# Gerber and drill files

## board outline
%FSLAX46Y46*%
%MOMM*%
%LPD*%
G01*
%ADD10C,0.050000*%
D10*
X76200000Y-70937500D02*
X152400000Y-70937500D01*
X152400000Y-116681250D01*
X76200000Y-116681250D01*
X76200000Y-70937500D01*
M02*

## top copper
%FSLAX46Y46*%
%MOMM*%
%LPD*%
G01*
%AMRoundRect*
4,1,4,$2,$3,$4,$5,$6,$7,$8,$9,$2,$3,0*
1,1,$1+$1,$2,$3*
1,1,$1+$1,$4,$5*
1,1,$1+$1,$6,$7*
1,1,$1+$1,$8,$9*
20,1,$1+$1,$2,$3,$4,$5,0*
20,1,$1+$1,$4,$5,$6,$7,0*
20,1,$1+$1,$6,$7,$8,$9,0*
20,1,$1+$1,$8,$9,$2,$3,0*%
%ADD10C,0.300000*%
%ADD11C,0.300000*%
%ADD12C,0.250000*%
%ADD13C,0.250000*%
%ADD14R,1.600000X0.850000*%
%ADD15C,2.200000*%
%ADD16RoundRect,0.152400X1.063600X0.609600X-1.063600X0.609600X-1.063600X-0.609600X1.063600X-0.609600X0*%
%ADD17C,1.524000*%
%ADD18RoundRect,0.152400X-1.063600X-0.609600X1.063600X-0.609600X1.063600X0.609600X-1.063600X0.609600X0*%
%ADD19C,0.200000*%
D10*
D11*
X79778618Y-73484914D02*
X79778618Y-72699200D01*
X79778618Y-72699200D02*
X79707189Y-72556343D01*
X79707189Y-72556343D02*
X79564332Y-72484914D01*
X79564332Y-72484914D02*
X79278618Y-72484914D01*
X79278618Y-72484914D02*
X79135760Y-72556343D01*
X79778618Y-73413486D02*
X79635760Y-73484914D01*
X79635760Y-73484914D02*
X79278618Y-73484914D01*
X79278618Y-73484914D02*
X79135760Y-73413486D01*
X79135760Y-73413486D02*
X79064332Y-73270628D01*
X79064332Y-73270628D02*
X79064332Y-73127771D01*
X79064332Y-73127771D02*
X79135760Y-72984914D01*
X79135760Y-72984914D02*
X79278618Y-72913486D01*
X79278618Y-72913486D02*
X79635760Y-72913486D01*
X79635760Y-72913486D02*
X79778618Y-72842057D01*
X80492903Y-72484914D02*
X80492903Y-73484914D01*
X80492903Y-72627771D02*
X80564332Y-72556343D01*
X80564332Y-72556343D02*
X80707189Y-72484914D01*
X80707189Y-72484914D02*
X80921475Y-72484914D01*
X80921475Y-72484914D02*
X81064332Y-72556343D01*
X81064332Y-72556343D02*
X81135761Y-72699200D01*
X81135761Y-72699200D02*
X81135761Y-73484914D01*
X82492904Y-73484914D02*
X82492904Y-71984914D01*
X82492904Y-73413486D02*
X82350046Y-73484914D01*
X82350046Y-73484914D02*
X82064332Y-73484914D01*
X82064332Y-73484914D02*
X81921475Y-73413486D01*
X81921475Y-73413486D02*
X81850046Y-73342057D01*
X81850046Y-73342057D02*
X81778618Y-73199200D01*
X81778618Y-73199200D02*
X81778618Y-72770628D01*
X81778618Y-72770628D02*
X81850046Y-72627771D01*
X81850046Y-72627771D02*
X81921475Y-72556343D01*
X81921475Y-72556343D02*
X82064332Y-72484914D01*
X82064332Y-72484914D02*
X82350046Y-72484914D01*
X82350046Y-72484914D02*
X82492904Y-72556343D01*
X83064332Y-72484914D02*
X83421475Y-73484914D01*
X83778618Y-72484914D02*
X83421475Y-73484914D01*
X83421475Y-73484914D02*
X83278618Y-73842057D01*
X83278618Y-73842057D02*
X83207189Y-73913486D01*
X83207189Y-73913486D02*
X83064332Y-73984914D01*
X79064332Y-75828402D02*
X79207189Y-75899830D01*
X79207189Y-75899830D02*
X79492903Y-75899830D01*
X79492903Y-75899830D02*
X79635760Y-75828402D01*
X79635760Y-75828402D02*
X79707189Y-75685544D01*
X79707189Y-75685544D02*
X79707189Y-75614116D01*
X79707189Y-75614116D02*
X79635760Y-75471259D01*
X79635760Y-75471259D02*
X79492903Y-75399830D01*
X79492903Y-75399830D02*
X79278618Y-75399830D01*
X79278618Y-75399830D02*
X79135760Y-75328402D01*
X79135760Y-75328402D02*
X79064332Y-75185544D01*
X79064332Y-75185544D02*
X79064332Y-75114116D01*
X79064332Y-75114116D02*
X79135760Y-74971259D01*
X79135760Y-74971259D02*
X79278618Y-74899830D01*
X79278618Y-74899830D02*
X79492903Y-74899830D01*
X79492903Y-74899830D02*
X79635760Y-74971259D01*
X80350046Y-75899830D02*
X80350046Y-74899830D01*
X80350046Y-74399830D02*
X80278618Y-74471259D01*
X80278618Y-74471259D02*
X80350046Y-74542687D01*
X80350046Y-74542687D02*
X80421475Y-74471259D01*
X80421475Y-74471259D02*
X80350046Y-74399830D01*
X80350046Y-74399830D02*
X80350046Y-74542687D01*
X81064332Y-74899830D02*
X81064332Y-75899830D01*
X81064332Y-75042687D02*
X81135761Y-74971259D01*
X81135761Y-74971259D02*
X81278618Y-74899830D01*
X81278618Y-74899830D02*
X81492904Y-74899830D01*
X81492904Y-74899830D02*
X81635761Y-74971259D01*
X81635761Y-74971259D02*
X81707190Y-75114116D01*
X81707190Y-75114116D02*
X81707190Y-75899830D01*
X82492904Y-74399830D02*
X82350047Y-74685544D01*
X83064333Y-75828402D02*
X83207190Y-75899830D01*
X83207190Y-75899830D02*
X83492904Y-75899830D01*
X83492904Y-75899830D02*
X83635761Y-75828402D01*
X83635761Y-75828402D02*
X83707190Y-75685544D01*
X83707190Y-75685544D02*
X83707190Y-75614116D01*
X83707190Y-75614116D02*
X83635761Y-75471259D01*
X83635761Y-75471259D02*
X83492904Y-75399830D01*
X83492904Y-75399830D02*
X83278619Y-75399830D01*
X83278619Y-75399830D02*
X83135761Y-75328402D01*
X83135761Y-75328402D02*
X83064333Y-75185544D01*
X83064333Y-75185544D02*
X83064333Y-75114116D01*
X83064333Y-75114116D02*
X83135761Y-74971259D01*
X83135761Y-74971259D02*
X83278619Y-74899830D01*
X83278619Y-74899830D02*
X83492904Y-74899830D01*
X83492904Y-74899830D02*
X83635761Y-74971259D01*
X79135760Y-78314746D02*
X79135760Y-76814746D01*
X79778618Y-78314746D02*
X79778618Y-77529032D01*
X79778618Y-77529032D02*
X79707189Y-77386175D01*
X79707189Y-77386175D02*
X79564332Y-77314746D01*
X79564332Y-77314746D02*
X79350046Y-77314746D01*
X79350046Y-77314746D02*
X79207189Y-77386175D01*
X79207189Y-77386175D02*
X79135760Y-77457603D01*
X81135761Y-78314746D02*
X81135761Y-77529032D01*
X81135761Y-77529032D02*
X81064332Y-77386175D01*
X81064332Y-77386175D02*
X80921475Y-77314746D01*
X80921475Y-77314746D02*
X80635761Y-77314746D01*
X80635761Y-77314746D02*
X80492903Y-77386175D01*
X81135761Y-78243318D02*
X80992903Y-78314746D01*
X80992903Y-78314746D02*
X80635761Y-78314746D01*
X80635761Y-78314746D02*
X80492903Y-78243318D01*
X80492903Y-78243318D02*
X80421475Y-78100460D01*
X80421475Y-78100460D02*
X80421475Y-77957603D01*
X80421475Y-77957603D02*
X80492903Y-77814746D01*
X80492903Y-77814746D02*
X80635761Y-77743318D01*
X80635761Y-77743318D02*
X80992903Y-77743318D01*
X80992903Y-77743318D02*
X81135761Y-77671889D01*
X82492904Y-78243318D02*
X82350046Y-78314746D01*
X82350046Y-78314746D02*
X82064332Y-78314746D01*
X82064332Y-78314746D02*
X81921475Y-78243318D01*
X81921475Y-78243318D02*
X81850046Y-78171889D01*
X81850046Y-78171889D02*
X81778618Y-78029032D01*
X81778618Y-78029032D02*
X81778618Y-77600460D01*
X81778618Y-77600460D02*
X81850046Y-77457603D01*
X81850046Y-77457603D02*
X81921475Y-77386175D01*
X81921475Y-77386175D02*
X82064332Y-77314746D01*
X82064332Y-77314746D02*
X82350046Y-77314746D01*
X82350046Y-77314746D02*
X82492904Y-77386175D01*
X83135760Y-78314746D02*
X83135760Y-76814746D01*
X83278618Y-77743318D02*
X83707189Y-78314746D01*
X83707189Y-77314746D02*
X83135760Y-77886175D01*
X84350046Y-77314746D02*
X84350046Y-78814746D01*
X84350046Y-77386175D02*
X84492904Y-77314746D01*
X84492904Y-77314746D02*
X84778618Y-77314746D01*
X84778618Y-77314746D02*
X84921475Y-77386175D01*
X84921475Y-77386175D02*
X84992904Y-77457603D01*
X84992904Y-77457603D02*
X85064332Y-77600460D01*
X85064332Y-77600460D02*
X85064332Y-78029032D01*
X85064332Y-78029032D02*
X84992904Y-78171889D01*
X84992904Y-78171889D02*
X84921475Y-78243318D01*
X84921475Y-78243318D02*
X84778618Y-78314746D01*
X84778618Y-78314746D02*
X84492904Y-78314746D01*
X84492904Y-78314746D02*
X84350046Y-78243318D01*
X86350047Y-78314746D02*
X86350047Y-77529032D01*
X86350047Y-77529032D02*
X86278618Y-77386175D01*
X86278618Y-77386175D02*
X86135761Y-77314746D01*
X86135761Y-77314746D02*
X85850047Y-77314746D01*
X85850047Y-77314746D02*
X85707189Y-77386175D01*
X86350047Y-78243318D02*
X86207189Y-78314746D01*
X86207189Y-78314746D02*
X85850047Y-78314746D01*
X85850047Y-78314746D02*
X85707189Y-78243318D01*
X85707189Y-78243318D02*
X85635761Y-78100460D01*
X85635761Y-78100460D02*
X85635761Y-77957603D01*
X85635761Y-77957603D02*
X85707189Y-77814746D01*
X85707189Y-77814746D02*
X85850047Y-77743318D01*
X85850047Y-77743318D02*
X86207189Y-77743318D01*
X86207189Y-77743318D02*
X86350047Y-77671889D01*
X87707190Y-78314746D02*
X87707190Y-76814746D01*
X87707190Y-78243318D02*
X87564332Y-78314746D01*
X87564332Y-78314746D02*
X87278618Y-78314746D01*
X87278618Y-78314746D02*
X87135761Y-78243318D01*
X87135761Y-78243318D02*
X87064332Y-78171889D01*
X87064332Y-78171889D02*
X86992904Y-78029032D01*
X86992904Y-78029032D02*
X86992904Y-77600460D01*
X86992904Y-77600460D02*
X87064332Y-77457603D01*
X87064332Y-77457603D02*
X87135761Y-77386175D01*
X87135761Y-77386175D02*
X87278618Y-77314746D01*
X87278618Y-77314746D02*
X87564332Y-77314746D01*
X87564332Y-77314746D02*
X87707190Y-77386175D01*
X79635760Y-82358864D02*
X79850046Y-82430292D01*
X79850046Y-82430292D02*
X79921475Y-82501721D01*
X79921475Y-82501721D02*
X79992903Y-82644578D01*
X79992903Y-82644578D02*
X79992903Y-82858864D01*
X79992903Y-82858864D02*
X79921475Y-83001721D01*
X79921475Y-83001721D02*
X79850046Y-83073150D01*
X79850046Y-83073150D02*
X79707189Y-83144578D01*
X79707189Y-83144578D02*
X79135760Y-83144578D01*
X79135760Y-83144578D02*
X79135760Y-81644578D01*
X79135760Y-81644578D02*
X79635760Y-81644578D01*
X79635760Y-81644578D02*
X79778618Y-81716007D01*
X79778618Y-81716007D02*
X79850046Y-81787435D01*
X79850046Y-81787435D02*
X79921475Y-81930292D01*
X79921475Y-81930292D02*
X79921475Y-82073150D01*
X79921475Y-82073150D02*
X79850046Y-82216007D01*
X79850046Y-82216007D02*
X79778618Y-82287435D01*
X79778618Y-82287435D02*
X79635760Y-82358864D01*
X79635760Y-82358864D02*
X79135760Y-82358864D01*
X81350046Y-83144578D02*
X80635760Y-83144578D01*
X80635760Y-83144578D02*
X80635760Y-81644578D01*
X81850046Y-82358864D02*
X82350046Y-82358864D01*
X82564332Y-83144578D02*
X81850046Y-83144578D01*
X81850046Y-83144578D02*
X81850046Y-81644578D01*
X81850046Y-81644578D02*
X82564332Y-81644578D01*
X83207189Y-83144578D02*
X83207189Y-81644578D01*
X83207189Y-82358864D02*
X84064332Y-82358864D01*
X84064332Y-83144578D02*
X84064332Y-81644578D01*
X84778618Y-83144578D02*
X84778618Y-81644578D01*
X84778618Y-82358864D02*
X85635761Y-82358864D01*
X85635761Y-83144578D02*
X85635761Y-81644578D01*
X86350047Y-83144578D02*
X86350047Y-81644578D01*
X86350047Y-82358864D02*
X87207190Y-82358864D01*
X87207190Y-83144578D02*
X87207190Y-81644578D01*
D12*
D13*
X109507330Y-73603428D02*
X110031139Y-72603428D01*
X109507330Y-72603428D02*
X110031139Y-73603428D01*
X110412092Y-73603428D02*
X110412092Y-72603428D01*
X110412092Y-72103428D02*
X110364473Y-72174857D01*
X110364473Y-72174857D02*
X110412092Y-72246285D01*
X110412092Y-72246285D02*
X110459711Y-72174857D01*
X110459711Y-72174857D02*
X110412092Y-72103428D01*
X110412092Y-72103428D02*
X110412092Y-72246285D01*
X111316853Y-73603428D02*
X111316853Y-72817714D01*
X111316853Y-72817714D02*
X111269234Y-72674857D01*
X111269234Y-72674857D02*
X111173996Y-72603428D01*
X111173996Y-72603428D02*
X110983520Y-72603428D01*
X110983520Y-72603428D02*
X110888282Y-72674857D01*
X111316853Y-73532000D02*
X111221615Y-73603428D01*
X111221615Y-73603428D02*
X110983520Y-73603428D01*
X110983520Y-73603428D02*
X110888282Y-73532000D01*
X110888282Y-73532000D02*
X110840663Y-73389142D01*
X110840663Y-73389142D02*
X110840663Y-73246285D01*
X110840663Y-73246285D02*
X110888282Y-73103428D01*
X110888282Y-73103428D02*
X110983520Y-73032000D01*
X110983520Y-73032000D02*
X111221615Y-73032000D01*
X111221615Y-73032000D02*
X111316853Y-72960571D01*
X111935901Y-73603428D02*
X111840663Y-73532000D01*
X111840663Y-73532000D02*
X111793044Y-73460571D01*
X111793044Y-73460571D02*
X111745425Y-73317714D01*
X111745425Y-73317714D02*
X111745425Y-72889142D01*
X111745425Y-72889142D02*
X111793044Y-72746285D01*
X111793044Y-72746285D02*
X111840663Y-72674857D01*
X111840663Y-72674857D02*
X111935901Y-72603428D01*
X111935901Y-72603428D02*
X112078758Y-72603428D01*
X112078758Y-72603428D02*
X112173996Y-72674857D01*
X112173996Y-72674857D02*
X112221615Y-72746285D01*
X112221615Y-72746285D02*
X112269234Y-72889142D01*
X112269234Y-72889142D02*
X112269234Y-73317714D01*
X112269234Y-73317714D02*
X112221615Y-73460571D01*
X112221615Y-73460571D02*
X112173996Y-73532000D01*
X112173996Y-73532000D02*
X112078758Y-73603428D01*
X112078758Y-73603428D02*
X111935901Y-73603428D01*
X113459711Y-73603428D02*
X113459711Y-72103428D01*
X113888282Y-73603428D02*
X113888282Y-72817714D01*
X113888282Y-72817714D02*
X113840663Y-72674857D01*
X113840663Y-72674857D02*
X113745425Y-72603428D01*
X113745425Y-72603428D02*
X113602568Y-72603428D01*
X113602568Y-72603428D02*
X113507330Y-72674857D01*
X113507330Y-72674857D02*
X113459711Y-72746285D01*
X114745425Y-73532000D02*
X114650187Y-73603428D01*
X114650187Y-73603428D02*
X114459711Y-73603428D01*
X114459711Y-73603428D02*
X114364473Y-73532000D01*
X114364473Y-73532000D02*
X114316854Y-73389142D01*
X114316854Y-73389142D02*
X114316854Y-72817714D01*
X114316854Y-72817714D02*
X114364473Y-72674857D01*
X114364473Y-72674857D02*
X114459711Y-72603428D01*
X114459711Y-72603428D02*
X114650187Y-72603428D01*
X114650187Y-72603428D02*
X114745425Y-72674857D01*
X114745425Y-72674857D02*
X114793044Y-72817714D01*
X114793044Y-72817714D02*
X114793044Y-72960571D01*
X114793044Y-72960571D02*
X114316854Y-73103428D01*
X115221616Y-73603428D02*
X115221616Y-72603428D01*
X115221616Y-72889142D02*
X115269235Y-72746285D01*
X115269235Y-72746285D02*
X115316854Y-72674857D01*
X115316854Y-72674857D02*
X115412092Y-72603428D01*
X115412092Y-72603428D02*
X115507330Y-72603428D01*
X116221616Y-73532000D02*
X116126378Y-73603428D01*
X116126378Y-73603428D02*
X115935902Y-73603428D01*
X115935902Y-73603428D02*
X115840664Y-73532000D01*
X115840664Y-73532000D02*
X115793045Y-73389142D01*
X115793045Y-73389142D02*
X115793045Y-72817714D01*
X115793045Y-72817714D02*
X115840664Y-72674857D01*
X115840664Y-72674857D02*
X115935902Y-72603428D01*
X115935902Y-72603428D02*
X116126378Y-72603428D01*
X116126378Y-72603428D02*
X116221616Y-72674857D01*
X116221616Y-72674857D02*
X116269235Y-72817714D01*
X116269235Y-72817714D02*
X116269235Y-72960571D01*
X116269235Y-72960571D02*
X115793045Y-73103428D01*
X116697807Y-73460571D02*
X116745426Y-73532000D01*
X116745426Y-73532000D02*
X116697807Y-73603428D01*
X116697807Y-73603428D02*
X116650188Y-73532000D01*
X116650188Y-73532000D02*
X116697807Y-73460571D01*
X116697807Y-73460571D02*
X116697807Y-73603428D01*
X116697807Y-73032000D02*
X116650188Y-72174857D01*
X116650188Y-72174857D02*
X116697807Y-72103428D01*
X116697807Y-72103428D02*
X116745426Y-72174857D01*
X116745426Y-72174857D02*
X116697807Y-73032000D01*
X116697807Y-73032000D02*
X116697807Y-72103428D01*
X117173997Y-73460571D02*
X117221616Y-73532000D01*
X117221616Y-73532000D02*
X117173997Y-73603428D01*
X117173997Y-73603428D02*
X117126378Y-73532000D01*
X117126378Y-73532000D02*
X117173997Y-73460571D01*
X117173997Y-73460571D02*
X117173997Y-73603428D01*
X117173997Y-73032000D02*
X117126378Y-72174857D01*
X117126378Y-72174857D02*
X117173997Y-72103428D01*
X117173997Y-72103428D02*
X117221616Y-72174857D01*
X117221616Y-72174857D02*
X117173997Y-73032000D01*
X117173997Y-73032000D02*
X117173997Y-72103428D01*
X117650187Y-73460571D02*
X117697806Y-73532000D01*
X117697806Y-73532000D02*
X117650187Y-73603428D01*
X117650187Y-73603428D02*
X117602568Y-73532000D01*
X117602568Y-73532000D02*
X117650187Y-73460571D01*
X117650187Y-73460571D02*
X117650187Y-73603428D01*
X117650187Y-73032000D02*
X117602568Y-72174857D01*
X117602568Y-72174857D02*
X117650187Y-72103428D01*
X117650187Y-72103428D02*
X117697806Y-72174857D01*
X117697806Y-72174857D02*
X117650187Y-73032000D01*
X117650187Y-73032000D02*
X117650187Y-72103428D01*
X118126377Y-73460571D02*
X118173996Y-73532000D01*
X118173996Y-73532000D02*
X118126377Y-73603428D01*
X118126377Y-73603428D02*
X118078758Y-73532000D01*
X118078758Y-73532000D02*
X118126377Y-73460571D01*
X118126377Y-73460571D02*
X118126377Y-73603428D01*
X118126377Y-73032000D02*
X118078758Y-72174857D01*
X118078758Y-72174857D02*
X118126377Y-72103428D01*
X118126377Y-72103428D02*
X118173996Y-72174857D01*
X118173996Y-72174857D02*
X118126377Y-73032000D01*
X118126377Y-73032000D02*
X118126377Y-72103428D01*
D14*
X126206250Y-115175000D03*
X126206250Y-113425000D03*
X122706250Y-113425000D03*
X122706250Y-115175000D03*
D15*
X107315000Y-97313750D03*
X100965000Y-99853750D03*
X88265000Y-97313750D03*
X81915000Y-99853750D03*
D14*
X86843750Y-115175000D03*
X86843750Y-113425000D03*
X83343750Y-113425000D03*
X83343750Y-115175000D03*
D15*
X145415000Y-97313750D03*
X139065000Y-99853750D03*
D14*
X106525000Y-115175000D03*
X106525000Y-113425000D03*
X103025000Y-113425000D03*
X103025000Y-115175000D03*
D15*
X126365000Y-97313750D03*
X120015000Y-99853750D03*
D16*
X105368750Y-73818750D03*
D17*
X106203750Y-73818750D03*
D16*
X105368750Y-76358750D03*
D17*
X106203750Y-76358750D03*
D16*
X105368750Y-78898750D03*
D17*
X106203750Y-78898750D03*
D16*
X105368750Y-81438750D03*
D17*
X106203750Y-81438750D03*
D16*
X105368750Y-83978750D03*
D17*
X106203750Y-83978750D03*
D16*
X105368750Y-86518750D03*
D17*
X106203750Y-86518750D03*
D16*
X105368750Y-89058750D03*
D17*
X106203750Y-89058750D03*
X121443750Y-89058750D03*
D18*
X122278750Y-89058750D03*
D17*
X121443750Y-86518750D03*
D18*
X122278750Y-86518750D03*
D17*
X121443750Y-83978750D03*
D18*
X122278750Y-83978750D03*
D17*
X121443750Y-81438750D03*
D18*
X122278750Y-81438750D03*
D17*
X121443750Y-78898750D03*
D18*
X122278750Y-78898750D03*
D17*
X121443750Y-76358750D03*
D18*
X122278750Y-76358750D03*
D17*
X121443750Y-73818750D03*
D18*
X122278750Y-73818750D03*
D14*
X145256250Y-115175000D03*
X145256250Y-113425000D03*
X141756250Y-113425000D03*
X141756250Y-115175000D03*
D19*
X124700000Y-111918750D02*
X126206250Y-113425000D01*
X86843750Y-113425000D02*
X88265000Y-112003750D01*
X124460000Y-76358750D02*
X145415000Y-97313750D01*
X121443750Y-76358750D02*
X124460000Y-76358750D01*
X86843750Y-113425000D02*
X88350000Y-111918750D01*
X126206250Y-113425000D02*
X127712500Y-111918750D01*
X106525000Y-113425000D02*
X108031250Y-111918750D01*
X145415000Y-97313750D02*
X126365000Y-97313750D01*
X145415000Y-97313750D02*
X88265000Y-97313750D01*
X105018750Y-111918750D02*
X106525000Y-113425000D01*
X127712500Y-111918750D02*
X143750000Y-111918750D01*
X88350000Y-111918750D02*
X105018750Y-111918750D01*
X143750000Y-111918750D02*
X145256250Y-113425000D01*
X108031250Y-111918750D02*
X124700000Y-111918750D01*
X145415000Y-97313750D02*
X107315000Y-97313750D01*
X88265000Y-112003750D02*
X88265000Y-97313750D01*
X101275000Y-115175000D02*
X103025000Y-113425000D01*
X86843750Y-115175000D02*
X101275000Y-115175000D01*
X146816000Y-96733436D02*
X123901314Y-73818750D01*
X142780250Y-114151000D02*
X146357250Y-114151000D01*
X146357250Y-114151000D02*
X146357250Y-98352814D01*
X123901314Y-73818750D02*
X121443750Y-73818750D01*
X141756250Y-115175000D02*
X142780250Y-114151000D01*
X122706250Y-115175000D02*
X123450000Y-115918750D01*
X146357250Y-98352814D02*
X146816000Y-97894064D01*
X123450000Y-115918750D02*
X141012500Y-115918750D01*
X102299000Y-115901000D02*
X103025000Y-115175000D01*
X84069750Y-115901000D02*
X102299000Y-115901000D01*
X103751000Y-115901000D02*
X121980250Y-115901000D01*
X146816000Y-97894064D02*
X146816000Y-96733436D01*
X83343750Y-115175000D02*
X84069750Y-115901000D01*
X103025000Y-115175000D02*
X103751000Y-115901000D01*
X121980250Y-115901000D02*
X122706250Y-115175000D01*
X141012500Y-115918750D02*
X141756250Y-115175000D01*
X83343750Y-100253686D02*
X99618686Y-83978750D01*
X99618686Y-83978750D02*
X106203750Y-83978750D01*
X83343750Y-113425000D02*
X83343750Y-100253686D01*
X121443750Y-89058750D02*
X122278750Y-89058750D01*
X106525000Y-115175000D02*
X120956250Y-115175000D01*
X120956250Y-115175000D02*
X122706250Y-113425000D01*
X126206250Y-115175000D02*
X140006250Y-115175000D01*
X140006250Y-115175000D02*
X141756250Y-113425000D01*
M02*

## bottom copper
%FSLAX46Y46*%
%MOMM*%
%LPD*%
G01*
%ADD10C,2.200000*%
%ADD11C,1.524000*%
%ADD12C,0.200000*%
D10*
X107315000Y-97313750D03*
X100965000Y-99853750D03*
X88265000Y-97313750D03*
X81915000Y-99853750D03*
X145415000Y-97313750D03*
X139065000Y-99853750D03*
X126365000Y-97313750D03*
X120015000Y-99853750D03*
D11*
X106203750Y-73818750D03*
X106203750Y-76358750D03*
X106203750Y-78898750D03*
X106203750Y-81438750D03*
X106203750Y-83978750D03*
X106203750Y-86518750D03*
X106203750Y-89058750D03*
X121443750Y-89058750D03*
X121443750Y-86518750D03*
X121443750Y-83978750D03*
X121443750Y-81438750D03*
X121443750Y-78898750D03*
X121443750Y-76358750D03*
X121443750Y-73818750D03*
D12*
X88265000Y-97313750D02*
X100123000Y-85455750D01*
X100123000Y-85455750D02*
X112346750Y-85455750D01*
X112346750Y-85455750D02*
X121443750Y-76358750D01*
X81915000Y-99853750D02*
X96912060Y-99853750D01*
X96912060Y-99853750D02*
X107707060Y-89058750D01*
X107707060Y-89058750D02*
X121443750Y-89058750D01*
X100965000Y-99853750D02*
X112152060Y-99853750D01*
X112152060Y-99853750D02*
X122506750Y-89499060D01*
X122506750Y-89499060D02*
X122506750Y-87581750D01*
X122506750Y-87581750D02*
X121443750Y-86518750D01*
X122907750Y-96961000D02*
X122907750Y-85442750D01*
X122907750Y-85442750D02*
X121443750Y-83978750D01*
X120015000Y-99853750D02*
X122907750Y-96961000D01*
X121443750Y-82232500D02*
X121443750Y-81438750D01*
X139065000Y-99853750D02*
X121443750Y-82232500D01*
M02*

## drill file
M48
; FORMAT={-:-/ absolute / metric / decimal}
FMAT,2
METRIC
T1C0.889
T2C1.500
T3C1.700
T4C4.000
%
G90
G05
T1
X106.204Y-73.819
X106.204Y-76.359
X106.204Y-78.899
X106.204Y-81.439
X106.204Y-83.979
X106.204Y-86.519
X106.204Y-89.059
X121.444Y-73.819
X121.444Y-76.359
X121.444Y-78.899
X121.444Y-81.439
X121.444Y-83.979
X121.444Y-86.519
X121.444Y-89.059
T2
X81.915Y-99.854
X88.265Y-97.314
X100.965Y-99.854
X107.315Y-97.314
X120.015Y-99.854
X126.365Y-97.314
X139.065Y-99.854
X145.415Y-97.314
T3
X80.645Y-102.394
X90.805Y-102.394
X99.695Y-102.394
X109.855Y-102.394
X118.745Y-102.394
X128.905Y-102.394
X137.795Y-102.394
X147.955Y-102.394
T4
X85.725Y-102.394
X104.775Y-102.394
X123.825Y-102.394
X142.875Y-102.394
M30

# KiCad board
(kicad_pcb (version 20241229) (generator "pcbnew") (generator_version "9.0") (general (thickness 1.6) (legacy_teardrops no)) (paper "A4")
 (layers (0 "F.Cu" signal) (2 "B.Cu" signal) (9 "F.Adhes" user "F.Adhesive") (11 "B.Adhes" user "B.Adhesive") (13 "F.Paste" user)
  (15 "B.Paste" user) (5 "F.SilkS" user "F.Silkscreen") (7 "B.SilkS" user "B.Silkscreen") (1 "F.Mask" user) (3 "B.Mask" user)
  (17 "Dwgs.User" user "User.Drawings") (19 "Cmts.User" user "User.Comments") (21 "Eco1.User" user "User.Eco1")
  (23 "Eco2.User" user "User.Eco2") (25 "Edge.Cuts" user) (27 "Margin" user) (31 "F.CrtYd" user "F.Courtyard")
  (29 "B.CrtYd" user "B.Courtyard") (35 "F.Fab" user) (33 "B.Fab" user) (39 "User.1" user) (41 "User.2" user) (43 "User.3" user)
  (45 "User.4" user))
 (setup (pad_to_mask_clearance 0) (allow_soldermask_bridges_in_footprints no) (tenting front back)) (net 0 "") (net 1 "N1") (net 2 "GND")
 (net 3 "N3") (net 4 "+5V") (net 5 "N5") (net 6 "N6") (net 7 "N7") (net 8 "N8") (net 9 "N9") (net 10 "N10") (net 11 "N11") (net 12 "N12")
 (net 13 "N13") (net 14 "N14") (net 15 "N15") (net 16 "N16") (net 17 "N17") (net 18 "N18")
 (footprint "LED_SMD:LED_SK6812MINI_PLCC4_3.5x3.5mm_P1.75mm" (layer "F.Cu") (at 124.45625 114.3 180)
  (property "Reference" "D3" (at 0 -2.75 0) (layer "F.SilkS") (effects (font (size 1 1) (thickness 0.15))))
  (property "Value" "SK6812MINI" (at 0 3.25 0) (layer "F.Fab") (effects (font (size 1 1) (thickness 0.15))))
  (pad "1" smd rect (at -1.75 -0.875 180) (size 1.6 0.85) (layers "F.Cu" "F.Mask" "F.Paste") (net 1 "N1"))
  (pad "2" smd rect (at -1.75 0.875 180) (size 1.6 0.85) (layers "F.Cu" "F.Mask" "F.Paste") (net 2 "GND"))
  (pad "3" smd rect (at 1.75 0.875 180) (size 1.6 0.85) (layers "F.Cu" "F.Mask" "F.Paste") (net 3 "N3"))
  (pad "4" smd rect (at 1.75 -0.875 180) (size 1.6 0.85) (layers "F.Cu" "F.Mask" "F.Paste") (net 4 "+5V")))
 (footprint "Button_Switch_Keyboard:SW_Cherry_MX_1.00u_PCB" (layer "F.Cu") (at 107.315 97.31375)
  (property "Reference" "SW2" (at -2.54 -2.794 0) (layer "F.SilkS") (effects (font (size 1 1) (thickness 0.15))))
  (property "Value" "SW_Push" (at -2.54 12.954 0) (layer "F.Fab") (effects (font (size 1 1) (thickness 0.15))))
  (pad "" np_thru_hole circle (at -7.62 5.08) (size 1.7 1.7) (drill 1.7) (layers "*.Cu" "*.Mask"))
  (pad "" np_thru_hole circle (at -2.54 5.08) (size 4 4) (drill 4) (layers "*.Cu" "*.Mask"))
  (pad "" np_thru_hole circle (at 2.54 5.08) (size 1.7 1.7) (drill 1.7) (layers "*.Cu" "*.Mask"))
  (pad "1" thru_hole circle (at 0 0) (size 2.2 2.2) (drill 1.5) (layers "*.Cu" "*.Mask") (remove_unused_layers no) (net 2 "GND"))
  (pad "2" thru_hole circle (at -6.35 2.54) (size 2.2 2.2) (drill 1.5) (layers "*.Cu" "*.Mask") (remove_unused_layers no) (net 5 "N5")))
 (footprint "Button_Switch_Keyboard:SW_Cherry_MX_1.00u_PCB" (layer "F.Cu") (at 88.265 97.31375)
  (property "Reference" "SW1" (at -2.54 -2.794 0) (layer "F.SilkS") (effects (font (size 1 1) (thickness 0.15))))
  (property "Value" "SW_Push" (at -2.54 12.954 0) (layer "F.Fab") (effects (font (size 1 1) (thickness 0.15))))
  (pad "" np_thru_hole circle (at -7.62 5.08) (size 1.7 1.7) (drill 1.7) (layers "*.Cu" "*.Mask"))
  (pad "" np_thru_hole circle (at -2.54 5.08) (size 4 4) (drill 4) (layers "*.Cu" "*.Mask"))
  (pad "" np_thru_hole circle (at 2.54 5.08) (size 1.7 1.7) (drill 1.7) (layers "*.Cu" "*.Mask"))
  (pad "1" thru_hole circle (at 0 0) (size 2.2 2.2) (drill 1.5) (layers "*.Cu" "*.Mask") (remove_unused_layers no) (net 2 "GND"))
  (pad "2" thru_hole circle (at -6.35 2.54) (size 2.2 2.2) (drill 1.5) (layers "*.Cu" "*.Mask") (remove_unused_layers no) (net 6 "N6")))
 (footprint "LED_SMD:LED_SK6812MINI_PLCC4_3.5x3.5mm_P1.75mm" (layer "F.Cu") (at 85.09375 114.3 180)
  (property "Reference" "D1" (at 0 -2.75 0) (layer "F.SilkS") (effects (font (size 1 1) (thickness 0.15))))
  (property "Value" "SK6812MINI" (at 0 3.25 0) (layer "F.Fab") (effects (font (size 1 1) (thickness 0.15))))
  (pad "1" smd rect (at -1.75 -0.875 180) (size 1.6 0.85) (layers "F.Cu" "F.Mask" "F.Paste") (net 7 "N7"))
  (pad "2" smd rect (at -1.75 0.875 180) (size 1.6 0.85) (layers "F.Cu" "F.Mask" "F.Paste") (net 2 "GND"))
  (pad "3" smd rect (at 1.75 0.875 180) (size 1.6 0.85) (layers "F.Cu" "F.Mask" "F.Paste") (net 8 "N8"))
  (pad "4" smd rect (at 1.75 -0.875 180) (size 1.6 0.85) (layers "F.Cu" "F.Mask" "F.Paste") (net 4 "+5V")))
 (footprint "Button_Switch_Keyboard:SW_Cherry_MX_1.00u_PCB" (layer "F.Cu") (at 145.415 97.31375)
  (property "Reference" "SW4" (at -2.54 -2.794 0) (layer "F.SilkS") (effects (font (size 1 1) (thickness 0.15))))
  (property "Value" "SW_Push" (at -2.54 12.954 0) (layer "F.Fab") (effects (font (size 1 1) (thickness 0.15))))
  (pad "" np_thru_hole circle (at -7.62 5.08) (size 1.7 1.7) (drill 1.7) (layers "*.Cu" "*.Mask"))
  (pad "" np_thru_hole circle (at -2.54 5.08) (size 4 4) (drill 4) (layers "*.Cu" "*.Mask"))
  (pad "" np_thru_hole circle (at 2.54 5.08) (size 1.7 1.7) (drill 1.7) (layers "*.Cu" "*.Mask"))
  (pad "1" thru_hole circle (at 0 0) (size 2.2 2.2) (drill 1.5) (layers "*.Cu" "*.Mask") (remove_unused_layers no) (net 2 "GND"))
  (pad "2" thru_hole circle (at -6.35 2.54) (size 2.2 2.2) (drill 1.5) (layers "*.Cu" "*.Mask") (remove_unused_layers no) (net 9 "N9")))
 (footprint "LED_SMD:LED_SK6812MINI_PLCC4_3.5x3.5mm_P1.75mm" (layer "F.Cu") (at 104.775 114.3 180)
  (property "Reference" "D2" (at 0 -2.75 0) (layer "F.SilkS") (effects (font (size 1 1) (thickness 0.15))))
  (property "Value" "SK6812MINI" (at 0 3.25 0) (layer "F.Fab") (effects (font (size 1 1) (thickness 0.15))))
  (pad "1" smd rect (at -1.75 -0.875 180) (size 1.6 0.85) (layers "F.Cu" "F.Mask" "F.Paste") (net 3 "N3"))
  (pad "2" smd rect (at -1.75 0.875 180) (size 1.6 0.85) (layers "F.Cu" "F.Mask" "F.Paste") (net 2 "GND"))
  (pad "3" smd rect (at 1.75 0.875 180) (size 1.6 0.85) (layers "F.Cu" "F.Mask" "F.Paste") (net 7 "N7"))
  (pad "4" smd rect (at 1.75 -0.875 180) (size 1.6 0.85) (layers "F.Cu" "F.Mask" "F.Paste") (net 4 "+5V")))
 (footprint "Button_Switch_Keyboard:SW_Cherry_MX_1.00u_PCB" (layer "F.Cu") (at 126.365 97.31375)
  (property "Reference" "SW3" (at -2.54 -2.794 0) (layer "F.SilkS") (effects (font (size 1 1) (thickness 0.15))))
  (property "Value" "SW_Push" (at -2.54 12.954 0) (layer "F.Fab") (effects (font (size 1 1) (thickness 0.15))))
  (pad "" np_thru_hole circle (at -7.62 5.08) (size 1.7 1.7) (drill 1.7) (layers "*.Cu" "*.Mask"))
  (pad "" np_thru_hole circle (at -2.54 5.08) (size 4 4) (drill 4) (layers "*.Cu" "*.Mask"))
  (pad "" np_thru_hole circle (at 2.54 5.08) (size 1.7 1.7) (drill 1.7) (layers "*.Cu" "*.Mask"))
  (pad "1" thru_hole circle (at 0 0) (size 2.2 2.2) (drill 1.5) (layers "*.Cu" "*.Mask") (remove_unused_layers no) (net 2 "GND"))
  (pad "2" thru_hole circle (at -6.35 2.54) (size 2.2 2.2) (drill 1.5) (layers "*.Cu" "*.Mask") (remove_unused_layers no) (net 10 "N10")))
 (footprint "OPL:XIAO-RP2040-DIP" (layer "F.Cu") (at 113.82375 81.43875)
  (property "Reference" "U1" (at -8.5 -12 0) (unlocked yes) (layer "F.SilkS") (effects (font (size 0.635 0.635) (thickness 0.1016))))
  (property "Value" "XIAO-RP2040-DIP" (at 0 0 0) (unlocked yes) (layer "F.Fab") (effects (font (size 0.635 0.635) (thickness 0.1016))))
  (pad "1" smd roundrect (at -8.455 -7.62 180) (size 2.432 1.524) (layers "F.Cu" "F.Mask") (roundrect_rratio 0.1) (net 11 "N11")
   (thermal_bridge_angle 45))
  (pad "1" thru_hole circle (at -7.62 -7.62 180) (size 1.524 1.524) (drill 0.889) (layers "*.Cu" "*.Mask") (remove_unused_layers no)
   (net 11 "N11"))
  (pad "2" smd roundrect (at -8.455 -5.08 180) (size 2.432 1.524) (layers "F.Cu" "F.Mask") (roundrect_rratio 0.1) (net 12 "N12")
   (thermal_bridge_angle 45))
  (pad "2" thru_hole circle (at -7.62 -5.08 180) (size 1.524 1.524) (drill 0.889) (layers "*.Cu" "*.Mask") (remove_unused_layers no)
   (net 12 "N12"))
  (pad "3" smd roundrect (at -8.455 -2.54 180) (size 2.432 1.524) (layers "F.Cu" "F.Mask") (roundrect_rratio 0.1) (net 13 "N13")
   (thermal_bridge_angle 45))
  (pad "3" thru_hole circle (at -7.62 -2.54 180) (size 1.524 1.524) (drill 0.889) (layers "*.Cu" "*.Mask") (remove_unused_layers no)
   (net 13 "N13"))
  (pad "4" smd roundrect (at -8.455 0 180) (size 2.432 1.524) (layers "F.Cu" "F.Mask") (roundrect_rratio 0.1) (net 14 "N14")
   (thermal_bridge_angle 45))
  (pad "4" thru_hole circle (at -7.62 0 180) (size 1.524 1.524) (drill 0.889) (layers "*.Cu" "*.Mask") (remove_unused_layers no)
   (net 14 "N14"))
  (pad "5" smd roundrect (at -8.455 2.54 180) (size 2.432 1.524) (layers "F.Cu" "F.Mask") (roundrect_rratio 0.1) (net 8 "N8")
   (thermal_bridge_angle 45))
  (pad "5" thru_hole circle (at -7.62 2.54 180) (size 1.524 1.524) (drill 0.889) (layers "*.Cu" "*.Mask") (remove_unused_layers no)
   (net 8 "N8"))
  (pad "6" smd roundrect (at -8.455 5.08 180) (size 2.432 1.524) (layers "F.Cu" "F.Mask") (roundrect_rratio 0.1) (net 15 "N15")
   (thermal_bridge_angle 45))
  (pad "6" thru_hole circle (at -7.62 5.08 180) (size 1.524 1.524) (drill 0.889) (layers "*.Cu" "*.Mask") (remove_unused_layers no)
   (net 15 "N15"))
  (pad "7" smd roundrect (at -8.455 7.62 180) (size 2.432 1.524) (layers "F.Cu" "F.Mask") (roundrect_rratio 0.1) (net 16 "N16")
   (thermal_bridge_angle 45))
  (pad "7" thru_hole circle (at -7.62 7.62 180) (size 1.524 1.524) (drill 0.889) (layers "*.Cu" "*.Mask") (remove_unused_layers no)
   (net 16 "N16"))
  (pad "8" thru_hole circle (at 7.62 7.62) (size 1.524 1.524) (drill 0.889) (layers "*.Cu" "*.Mask") (remove_unused_layers no) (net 6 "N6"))
  (pad "8" smd roundrect (at 8.455 7.62) (size 2.432 1.524) (layers "F.Cu" "F.Mask") (roundrect_rratio 0.1) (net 6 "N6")
   (thermal_bridge_angle 45))
  (pad "9" thru_hole circle (at 7.62 5.08) (size 1.524 1.524) (drill 0.889) (layers "*.Cu" "*.Mask") (remove_unused_layers no) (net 5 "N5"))
  (pad "9" smd roundrect (at 8.455 5.08) (size 2.432 1.524) (layers "F.Cu" "F.Mask") (roundrect_rratio 0.1) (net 5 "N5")
   (thermal_bridge_angle 45))
  (pad "10" thru_hole circle (at 7.62 2.54) (size 1.524 1.524) (drill 0.889) (layers "*.Cu" "*.Mask") (remove_unused_layers no)
   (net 10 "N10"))
  (pad "10" smd roundrect (at 8.455 2.54) (size 2.432 1.524) (layers "F.Cu" "F.Mask") (roundrect_rratio 0.1) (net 10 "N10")
   (thermal_bridge_angle 45))
  (pad "11" thru_hole circle (at 7.62 0) (size 1.524 1.524) (drill 0.889) (layers "*.Cu" "*.Mask") (remove_unused_layers no) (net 9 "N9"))
  (pad "11" smd roundrect (at 8.455 0) (size 2.432 1.524) (layers "F.Cu" "F.Mask") (roundrect_rratio 0.1) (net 9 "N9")
   (thermal_bridge_angle 45))
  (pad "12" thru_hole circle (at 7.62 -2.54) (size 1.524 1.524) (drill 0.889) (layers "*.Cu" "*.Mask") (remove_unused_layers no)
   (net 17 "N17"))
  (pad "12" smd roundrect (at 8.455 -2.54) (size 2.432 1.524) (layers "F.Cu" "F.Mask") (roundrect_rratio 0.1) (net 17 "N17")
   (thermal_bridge_angle 45))
  (pad "13" thru_hole circle (at 7.62 -5.08) (size 1.524 1.524) (drill 0.889) (layers "*.Cu" "*.Mask") (remove_unused_layers no)
   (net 2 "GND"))
  (pad "13" smd roundrect (at 8.455 -5.08) (size 2.432 1.524) (layers "F.Cu" "F.Mask") (roundrect_rratio 0.1) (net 2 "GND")
   (thermal_bridge_angle 45))
  (pad "14" thru_hole circle (at 7.62 -7.62) (size 1.524 1.524) (drill 0.889) (layers "*.Cu" "*.Mask") (remove_unused_layers no)
   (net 4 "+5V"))
  (pad "14" smd roundrect (at 8.455 -7.62) (size 2.432 1.524) (layers "F.Cu" "F.Mask") (roundrect_rratio 0.1) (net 4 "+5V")
   (thermal_bridge_angle 45)))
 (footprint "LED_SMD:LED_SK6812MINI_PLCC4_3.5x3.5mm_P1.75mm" (layer "F.Cu") (at 143.50625 114.3 180)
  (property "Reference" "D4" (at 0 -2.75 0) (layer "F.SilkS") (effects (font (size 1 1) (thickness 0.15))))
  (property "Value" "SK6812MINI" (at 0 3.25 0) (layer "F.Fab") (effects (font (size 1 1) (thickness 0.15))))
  (pad "1" smd rect (at -1.75 -0.875 180) (size 1.6 0.85) (layers "F.Cu" "F.Mask" "F.Paste") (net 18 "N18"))
  (pad "2" smd rect (at -1.75 0.875 180) (size 1.6 0.85) (layers "F.Cu" "F.Mask" "F.Paste") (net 2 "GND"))
  (pad "3" smd rect (at 1.75 0.875 180) (size 1.6 0.85) (layers "F.Cu" "F.Mask" "F.Paste") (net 1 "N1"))
  (pad "4" smd rect (at 1.75 -0.875 180) (size 1.6 0.85) (layers "F.Cu" "F.Mask" "F.Paste") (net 4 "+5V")))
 (gr_rect (start 76.2 70.9375) (end 152.4 116.68125) (stroke (width 0.05) (type default)) (fill no) (layer "Edge.Cuts"))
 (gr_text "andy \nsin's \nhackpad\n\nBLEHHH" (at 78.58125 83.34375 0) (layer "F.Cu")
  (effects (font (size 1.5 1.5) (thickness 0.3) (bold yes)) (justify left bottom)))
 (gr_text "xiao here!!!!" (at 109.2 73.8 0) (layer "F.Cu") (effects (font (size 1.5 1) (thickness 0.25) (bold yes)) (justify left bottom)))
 (segment (start 124.7 111.91875) (end 126.20625 113.425) (width 0.2) (layer "F.Cu") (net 2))
 (segment (start 86.84375 113.425) (end 88.265 112.00375) (width 0.2) (layer "F.Cu") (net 2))
 (segment (start 124.46 76.35875) (end 145.415 97.31375) (width 0.2) (layer "F.Cu") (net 2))
 (segment (start 121.44375 76.35875) (end 124.46 76.35875) (width 0.2) (layer "F.Cu") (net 2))
 (segment (start 86.84375 113.425) (end 88.35 111.91875) (width 0.2) (layer "F.Cu") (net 2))
 (segment (start 126.20625 113.425) (end 127.7125 111.91875) (width 0.2) (layer "F.Cu") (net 2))
 (segment (start 106.525 113.425) (end 108.03125 111.91875) (width 0.2) (layer "F.Cu") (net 2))
 (segment (start 145.415 97.31375) (end 126.365 97.31375) (width 0.2) (layer "F.Cu") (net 2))
 (segment (start 145.415 97.31375) (end 88.265 97.31375) (width 0.2) (layer "F.Cu") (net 2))
 (segment (start 105.01875 111.91875) (end 106.525 113.425) (width 0.2) (layer "F.Cu") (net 2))
 (segment (start 127.7125 111.91875) (end 143.75 111.91875) (width 0.2) (layer "F.Cu") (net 2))
 (segment (start 88.35 111.91875) (end 105.01875 111.91875) (width 0.2) (layer "F.Cu") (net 2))
 (segment (start 143.75 111.91875) (end 145.25625 113.425) (width 0.2) (layer "F.Cu") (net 2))
 (segment (start 108.03125 111.91875) (end 124.7 111.91875) (width 0.2) (layer "F.Cu") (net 2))
 (segment (start 145.415 97.31375) (end 107.315 97.31375) (width 0.2) (layer "F.Cu") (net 2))
 (segment (start 88.265 112.00375) (end 88.265 97.31375) (width 0.2) (layer "F.Cu") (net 2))
 (segment (start 88.265 97.31375) (end 100.123 85.45575) (width 0.2) (layer "B.Cu") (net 2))
 (segment (start 100.123 85.45575) (end 112.34675 85.45575) (width 0.2) (layer "B.Cu") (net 2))
 (segment (start 112.34675 85.45575) (end 121.44375 76.35875) (width 0.2) (layer "B.Cu") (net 2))
 (segment (start 101.275 115.175) (end 103.025 113.425) (width 0.2) (layer "F.Cu") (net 7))
 (segment (start 86.84375 115.175) (end 101.275 115.175) (width 0.2) (layer "F.Cu") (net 7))
 (segment (start 146.816 96.733436) (end 123.901314 73.81875) (width 0.2) (layer "F.Cu") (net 4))
 (segment (start 142.78025 114.151) (end 146.35725 114.151) (width 0.2) (layer "F.Cu") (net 4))
 (segment (start 146.35725 114.151) (end 146.35725 98.352814) (width 0.2) (layer "F.Cu") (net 4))
 (segment (start 123.901314 73.81875) (end 121.44375 73.81875) (width 0.2) (layer "F.Cu") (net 4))
 (segment (start 141.75625 115.175) (end 142.78025 114.151) (width 0.2) (layer "F.Cu") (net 4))
 (segment (start 122.70625 115.175) (end 123.45 115.91875) (width 0.2) (layer "F.Cu") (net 4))
 (segment (start 146.35725 98.352814) (end 146.816 97.894064) (width 0.2) (layer "F.Cu") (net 4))
 (segment (start 123.45 115.91875) (end 141.0125 115.91875) (width 0.2) (layer "F.Cu") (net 4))
 (segment (start 102.299 115.901) (end 103.025 115.175) (width 0.2) (layer "F.Cu") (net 4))
 (segment (start 84.06975 115.901) (end 102.299 115.901) (width 0.2) (layer "F.Cu") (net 4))
 (segment (start 103.751 115.901) (end 121.98025 115.901) (width 0.2) (layer "F.Cu") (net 4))
 (segment (start 146.816 97.894064) (end 146.816 96.733436) (width 0.2) (layer "F.Cu") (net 4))
 (segment (start 83.34375 115.175) (end 84.06975 115.901) (width 0.2) (layer "F.Cu") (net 4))
 (segment (start 103.025 115.175) (end 103.751 115.901) (width 0.2) (layer "F.Cu") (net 4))
 (segment (start 121.98025 115.901) (end 122.70625 115.175) (width 0.2) (layer "F.Cu") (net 4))
 (segment (start 141.0125 115.91875) (end 141.75625 115.175) (width 0.2) (layer "F.Cu") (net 4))
 (segment (start 83.34375 100.253686) (end 99.618686 83.97875) (width 0.2) (layer "F.Cu") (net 8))
 (segment (start 99.618686 83.97875) (end 106.20375 83.97875) (width 0.2) (layer "F.Cu") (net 8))
 (segment (start 83.34375 113.425) (end 83.34375 100.253686) (width 0.2) (layer "F.Cu") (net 8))
 (segment (start 121.44375 89.05875) (end 122.27875 89.05875) (width 0.2) (layer "F.Cu") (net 6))
 (segment (start 81.915 99.85375) (end 96.91206 99.85375) (width 0.2) (layer "B.Cu") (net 6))
 (segment (start 96.91206 99.85375) (end 107.70706 89.05875) (width 0.2) (layer "B.Cu") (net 6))
 (segment (start 107.70706 89.05875) (end 121.44375 89.05875) (width 0.2) (layer "B.Cu") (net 6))
 (segment (start 100.965 99.85375) (end 112.15206 99.85375) (width 0.2) (layer "B.Cu") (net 5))
 (segment (start 112.15206 99.85375) (end 122.50675 89.49906) (width 0.2) (layer "B.Cu") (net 5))
 (segment (start 122.50675 89.49906) (end 122.50675 87.58175) (width 0.2) (layer "B.Cu") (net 5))
 (segment (start 122.50675 87.58175) (end 121.44375 86.51875) (width 0.2) (layer "B.Cu") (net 5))
 (segment (start 122.90775 96.961) (end 122.90775 85.44275) (width 0.2) (layer "B.Cu") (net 10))
 (segment (start 122.90775 85.44275) (end 121.44375 83.97875) (width 0.2) (layer "B.Cu") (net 10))
 (segment (start 120.015 99.85375) (end 122.90775 96.961) (width 0.2) (layer "B.Cu") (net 10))
 (segment (start 121.44375 82.2325) (end 121.44375 81.43875) (width 0.2) (layer "B.Cu") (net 9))
 (segment (start 139.065 99.85375) (end 121.44375 82.2325) (width 0.2) (layer "B.Cu") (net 9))
 (segment (start 106.525 115.175) (end 120.95625 115.175) (width 0.2) (layer "F.Cu") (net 3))
 (segment (start 120.95625 115.175) (end 122.70625 113.425) (width 0.2) (layer "F.Cu") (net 3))
 (segment (start 126.20625 115.175) (end 140.00625 115.175) (width 0.2) (layer "F.Cu") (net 1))
 (segment (start 140.00625 115.175) (end 141.75625 113.425) (width 0.2) (layer "F.Cu") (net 1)))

